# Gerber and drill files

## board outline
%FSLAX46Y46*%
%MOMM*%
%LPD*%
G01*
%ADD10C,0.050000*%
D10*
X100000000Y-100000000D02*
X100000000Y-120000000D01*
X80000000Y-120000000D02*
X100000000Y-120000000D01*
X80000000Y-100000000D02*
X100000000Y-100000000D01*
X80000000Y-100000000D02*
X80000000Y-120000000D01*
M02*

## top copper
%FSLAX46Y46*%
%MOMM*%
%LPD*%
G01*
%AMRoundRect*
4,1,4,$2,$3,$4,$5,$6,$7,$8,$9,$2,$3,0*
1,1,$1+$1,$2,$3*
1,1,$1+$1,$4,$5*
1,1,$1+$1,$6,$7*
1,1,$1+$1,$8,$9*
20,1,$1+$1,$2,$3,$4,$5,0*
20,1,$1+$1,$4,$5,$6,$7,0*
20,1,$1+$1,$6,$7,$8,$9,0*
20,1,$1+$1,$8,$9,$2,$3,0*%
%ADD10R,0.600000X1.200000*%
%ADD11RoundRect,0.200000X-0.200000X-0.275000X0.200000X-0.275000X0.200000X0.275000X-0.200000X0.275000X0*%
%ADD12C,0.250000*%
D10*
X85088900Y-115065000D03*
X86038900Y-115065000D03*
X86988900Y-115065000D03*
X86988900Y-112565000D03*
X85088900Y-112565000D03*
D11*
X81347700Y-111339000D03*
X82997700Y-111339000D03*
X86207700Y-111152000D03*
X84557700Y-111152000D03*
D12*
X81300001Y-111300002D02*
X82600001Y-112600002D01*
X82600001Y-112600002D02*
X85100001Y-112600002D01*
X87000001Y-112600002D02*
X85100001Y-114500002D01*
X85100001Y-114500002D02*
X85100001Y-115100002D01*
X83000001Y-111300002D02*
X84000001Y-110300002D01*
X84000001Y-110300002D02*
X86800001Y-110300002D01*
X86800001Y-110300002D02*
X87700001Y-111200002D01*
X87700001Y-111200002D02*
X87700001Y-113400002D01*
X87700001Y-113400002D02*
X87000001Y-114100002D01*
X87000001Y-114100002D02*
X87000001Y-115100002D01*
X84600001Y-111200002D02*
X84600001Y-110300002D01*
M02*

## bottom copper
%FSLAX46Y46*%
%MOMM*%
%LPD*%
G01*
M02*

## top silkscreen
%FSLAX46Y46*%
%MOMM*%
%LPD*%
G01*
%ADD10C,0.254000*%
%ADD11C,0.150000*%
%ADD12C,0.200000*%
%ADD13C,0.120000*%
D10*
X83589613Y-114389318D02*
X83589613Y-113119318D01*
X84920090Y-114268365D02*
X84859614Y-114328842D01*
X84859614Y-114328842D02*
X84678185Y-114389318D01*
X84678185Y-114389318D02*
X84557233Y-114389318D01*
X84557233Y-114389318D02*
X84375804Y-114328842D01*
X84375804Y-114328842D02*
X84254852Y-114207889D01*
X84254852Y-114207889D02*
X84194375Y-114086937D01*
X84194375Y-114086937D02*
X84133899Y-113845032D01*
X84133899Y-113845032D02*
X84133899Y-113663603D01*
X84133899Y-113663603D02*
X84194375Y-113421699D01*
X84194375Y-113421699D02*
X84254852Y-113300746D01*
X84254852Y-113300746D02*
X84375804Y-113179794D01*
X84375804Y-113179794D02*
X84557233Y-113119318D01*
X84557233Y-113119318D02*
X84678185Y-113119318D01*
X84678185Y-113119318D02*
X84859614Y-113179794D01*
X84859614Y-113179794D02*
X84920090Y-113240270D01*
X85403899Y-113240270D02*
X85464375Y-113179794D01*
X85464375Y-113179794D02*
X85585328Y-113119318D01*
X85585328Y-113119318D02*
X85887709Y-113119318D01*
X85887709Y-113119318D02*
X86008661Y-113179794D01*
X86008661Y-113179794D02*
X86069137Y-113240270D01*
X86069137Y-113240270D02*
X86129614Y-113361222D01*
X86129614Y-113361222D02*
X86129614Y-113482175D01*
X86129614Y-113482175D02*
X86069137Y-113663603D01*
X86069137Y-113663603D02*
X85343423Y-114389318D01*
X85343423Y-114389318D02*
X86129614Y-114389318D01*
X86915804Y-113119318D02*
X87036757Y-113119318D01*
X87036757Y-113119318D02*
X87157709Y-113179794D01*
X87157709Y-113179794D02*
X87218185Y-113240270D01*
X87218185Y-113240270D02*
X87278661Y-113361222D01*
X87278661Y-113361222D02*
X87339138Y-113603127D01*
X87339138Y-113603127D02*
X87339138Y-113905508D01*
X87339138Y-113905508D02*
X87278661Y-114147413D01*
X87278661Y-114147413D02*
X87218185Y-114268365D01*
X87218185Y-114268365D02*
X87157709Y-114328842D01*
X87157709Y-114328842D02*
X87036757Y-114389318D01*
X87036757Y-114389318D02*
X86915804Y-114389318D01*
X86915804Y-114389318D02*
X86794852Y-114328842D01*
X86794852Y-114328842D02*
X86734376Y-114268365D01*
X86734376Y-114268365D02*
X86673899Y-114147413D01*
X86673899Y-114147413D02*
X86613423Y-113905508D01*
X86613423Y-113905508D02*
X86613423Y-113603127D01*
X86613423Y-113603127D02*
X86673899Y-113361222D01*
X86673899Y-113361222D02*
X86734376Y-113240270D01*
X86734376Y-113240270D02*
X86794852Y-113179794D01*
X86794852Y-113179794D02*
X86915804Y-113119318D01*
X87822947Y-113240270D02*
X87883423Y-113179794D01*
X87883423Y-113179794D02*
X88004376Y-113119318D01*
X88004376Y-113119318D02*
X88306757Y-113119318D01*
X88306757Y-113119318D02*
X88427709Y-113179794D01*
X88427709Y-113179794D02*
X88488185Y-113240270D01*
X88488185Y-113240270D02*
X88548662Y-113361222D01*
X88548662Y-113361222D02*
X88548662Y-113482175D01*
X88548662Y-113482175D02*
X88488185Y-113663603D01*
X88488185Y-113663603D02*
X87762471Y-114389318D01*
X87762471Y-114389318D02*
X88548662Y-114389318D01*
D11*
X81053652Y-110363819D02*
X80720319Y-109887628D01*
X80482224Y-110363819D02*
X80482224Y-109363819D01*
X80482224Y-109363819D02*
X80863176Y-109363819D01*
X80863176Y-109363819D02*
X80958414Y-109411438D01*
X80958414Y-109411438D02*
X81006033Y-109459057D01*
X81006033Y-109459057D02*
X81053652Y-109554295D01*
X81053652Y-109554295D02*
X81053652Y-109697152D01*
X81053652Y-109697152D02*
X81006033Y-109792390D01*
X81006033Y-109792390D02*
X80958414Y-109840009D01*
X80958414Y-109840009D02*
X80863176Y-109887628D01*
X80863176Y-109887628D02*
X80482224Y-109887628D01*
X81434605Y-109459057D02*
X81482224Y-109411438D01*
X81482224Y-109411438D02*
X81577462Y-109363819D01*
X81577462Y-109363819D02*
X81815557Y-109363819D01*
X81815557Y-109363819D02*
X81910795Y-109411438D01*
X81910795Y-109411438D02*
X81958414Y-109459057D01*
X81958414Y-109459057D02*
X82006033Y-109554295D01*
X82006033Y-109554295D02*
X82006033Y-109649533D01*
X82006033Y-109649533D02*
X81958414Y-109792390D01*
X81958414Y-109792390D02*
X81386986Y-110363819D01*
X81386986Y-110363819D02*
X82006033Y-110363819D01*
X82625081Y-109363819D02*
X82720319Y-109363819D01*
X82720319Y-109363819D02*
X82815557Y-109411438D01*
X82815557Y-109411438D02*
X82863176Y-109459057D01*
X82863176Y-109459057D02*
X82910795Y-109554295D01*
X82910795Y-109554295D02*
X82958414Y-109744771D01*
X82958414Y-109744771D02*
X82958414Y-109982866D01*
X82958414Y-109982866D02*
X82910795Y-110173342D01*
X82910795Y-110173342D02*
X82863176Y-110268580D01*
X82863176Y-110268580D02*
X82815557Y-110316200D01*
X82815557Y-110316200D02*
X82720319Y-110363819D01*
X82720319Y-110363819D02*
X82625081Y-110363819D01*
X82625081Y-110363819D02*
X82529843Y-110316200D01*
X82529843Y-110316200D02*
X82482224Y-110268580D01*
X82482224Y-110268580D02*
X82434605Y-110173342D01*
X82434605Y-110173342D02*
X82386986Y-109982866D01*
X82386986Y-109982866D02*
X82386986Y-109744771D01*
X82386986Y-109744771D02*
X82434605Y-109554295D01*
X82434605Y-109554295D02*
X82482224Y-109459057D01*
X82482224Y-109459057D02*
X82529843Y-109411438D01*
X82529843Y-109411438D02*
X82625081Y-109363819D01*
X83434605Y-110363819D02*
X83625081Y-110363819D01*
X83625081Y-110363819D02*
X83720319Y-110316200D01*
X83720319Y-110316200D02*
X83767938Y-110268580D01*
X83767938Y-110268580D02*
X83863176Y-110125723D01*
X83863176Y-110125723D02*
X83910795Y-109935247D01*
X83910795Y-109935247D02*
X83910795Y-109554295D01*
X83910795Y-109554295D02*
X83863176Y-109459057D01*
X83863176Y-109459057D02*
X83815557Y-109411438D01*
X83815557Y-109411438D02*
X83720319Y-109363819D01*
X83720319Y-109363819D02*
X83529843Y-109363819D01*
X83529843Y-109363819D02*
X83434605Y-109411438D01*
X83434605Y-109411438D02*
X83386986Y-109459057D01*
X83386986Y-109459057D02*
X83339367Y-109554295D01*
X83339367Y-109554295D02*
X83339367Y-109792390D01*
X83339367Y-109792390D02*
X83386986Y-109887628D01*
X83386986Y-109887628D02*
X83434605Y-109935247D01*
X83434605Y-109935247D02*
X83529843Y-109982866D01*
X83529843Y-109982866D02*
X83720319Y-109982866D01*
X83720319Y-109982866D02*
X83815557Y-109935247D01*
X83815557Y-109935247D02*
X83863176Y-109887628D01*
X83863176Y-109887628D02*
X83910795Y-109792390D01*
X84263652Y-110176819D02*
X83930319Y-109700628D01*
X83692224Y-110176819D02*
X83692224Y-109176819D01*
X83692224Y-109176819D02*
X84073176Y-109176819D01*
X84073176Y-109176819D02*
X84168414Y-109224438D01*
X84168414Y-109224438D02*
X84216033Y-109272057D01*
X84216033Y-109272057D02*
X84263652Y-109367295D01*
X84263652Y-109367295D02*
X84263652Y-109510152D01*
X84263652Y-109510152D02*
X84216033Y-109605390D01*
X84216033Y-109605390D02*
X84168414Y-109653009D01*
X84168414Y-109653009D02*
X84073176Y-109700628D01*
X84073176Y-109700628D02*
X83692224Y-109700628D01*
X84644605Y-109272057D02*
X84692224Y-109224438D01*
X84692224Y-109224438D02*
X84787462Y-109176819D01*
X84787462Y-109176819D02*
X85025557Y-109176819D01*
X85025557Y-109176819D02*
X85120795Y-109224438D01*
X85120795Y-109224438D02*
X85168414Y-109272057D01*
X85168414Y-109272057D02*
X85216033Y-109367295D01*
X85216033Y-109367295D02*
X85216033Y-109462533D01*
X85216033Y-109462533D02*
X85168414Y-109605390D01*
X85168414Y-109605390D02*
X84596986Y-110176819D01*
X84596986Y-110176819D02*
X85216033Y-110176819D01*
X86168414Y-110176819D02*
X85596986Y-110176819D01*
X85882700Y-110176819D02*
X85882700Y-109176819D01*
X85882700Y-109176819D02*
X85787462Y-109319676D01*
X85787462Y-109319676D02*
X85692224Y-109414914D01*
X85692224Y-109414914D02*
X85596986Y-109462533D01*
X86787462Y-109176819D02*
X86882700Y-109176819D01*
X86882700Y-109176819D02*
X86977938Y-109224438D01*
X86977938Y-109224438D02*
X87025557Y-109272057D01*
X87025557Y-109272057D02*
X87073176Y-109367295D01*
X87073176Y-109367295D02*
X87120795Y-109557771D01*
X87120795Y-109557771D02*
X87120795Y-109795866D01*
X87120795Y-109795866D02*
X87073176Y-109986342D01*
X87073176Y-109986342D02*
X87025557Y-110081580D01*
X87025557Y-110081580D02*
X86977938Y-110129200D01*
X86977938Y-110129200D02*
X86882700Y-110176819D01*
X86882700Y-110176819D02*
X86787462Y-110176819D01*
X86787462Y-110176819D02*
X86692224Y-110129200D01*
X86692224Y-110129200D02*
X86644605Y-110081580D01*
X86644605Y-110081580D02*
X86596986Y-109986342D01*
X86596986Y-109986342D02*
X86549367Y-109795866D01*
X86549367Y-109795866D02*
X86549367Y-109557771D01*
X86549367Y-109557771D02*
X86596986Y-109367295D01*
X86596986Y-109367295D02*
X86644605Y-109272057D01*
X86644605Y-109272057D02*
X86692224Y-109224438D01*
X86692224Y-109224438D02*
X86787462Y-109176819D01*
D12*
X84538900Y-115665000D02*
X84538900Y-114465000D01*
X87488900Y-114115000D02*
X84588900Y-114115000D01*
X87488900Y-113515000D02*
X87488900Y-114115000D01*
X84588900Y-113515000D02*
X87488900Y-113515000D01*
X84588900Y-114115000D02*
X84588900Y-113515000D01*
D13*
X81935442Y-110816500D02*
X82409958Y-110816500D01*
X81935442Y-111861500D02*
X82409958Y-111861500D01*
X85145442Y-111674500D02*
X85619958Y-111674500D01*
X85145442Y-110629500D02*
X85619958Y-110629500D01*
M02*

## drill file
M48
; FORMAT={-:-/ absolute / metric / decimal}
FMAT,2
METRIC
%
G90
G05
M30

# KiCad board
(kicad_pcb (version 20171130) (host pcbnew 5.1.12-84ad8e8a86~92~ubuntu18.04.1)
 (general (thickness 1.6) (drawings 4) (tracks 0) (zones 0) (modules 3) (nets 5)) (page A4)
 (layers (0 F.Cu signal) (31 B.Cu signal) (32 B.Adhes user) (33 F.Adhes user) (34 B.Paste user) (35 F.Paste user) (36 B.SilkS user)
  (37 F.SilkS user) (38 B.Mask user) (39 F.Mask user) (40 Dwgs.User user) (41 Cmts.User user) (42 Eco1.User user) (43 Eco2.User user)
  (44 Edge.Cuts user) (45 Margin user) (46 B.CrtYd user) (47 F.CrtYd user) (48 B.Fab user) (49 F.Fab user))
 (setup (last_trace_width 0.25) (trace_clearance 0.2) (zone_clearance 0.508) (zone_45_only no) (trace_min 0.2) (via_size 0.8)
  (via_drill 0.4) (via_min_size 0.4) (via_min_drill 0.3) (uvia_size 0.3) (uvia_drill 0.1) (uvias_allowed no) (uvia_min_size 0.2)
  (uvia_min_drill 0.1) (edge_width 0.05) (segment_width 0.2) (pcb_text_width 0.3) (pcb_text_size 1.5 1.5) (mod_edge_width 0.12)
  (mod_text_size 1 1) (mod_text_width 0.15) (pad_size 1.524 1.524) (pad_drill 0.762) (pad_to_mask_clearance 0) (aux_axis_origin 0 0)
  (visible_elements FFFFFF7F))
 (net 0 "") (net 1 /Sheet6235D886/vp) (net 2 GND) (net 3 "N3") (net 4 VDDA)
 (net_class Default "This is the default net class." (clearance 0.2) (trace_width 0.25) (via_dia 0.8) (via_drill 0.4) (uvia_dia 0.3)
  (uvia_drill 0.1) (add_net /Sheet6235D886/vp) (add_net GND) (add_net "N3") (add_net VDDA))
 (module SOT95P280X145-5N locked (layer F.Cu) (at 86.038900 113.815000 90.000000)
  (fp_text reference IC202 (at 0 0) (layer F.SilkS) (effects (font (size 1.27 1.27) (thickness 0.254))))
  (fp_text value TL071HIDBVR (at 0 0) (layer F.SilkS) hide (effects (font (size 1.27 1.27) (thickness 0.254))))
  (fp_line (start -1.85 -1.5) (end -0.65 -1.5) (layer F.SilkS) (width 0.2))
  (fp_line (start -0.3 1.45) (end -0.3 -1.45) (layer F.SilkS) (width 0.2))
  (fp_line (start 0.3 1.45) (end -0.3 1.45) (layer F.SilkS) (width 0.2))
  (fp_line (start 0.3 -1.45) (end 0.3 1.45) (layer F.SilkS) (width 0.2))
  (fp_line (start -0.3 -1.45) (end 0.3 -1.45) (layer F.SilkS) (width 0.2))
  (pad 1 smd rect (at -1.25 -0.95 180.000000) (size 0.6 1.2) (layers F.Cu F.Mask F.Paste) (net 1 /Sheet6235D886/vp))
  (pad 2 smd rect (at -1.25 0 180.000000) (size 0.6 1.2) (layers F.Cu F.Mask F.Paste) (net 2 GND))
  (pad 3 smd rect (at -1.25 0.95 180.000000) (size 0.6 1.2) (layers F.Cu F.Mask F.Paste) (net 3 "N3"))
  (pad 4 smd rect (at 1.25 0.95 180.000000) (size 0.6 1.2) (layers F.Cu F.Mask F.Paste) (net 1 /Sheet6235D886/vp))
  (pad 5 smd rect (at 1.25 -0.95 180.000000) (size 0.6 1.2) (layers F.Cu F.Mask F.Paste) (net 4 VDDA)))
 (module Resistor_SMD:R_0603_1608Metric (layer F.Cu) (at 82.172700 111.339000)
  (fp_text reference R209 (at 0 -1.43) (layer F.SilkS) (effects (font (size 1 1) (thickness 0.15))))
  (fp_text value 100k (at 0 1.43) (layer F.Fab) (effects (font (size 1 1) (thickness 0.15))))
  (fp_line (start -0.237258 -0.5225) (end 0.237258 -0.5225) (layer F.SilkS) (width 0.12))
  (fp_line (start -0.237258 0.5225) (end 0.237258 0.5225) (layer F.SilkS) (width 0.12))
  (pad 1 smd roundrect (at -0.825 0) (size 0.8 0.95) (layers F.Cu F.Mask F.Paste) (roundrect_rratio 0.25) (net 4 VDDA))
  (pad 2 smd roundrect (at 0.825 0) (size 0.8 0.95) (layers F.Cu F.Mask F.Paste) (roundrect_rratio 0.25) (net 3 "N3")))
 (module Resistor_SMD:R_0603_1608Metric (layer F.Cu) (at 85.382700 111.152000)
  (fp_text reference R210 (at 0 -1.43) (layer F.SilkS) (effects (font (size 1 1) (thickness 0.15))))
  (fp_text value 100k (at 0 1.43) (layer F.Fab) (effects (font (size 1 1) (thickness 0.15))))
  (fp_line (start -0.237258 0.5225) (end 0.237258 0.5225) (layer F.SilkS) (width 0.12))
  (fp_line (start -0.237258 -0.5225) (end 0.237258 -0.5225) (layer F.SilkS) (width 0.12))
  (pad 2 smd roundrect (at 0.825 0) (size 0.8 0.95) (layers F.Cu F.Mask F.Paste) (roundrect_rratio 0.25) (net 2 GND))
  (pad 1 smd roundrect (at -0.825 0) (size 0.8 0.95) (layers F.Cu F.Mask F.Paste) (roundrect_rratio 0.25) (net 3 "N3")))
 (gr_line (start 100 100) (end 100 120) (layer Edge.Cuts) (width 0.05))
 (gr_line (start 80 120) (end 100 120) (layer Edge.Cuts) (width 0.05))
 (gr_line (start 80 100) (end 100 100) (layer Edge.Cuts) (width 0.05))
 (gr_line (start 80 100) (end 80 120) (layer Edge.Cuts) (width 0.05))
 (segment (start 81.300001 111.300002) (end 82.600001 112.600002) (width 0.250000) (layer F.Cu) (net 4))
 (segment (start 82.600001 112.600002) (end 85.100001 112.600002) (width 0.250000) (layer F.Cu) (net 4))
 (segment (start 87.000001 112.600002) (end 85.100001 114.500002) (width 0.250000) (layer F.Cu) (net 1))
 (segment (start 85.100001 114.500002) (end 85.100001 115.100002) (width 0.250000) (layer F.Cu) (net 1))
 (segment (start 83.000001 111.300002) (end 84.000001 110.300002) (width 0.250000) (layer F.Cu) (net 3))
 (segment (start 84.000001 110.300002) (end 86.800001 110.300002) (width 0.250000) (layer F.Cu) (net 3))
 (segment (start 86.800001 110.300002) (end 87.700001 111.200002) (width 0.250000) (layer F.Cu) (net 3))
 (segment (start 87.700001 111.200002) (end 87.700001 113.400002) (width 0.250000) (layer F.Cu) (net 3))
 (segment (start 87.700001 113.400002) (end 87.000001 114.100002) (width 0.250000) (layer F.Cu) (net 3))
 (segment (start 87.000001 114.100002) (end 87.000001 115.100002) (width 0.250000) (layer F.Cu) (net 3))
 (segment (start 84.600001 111.200002) (end 84.600001 110.300002) (width 0.250000) (layer F.Cu) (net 3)))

